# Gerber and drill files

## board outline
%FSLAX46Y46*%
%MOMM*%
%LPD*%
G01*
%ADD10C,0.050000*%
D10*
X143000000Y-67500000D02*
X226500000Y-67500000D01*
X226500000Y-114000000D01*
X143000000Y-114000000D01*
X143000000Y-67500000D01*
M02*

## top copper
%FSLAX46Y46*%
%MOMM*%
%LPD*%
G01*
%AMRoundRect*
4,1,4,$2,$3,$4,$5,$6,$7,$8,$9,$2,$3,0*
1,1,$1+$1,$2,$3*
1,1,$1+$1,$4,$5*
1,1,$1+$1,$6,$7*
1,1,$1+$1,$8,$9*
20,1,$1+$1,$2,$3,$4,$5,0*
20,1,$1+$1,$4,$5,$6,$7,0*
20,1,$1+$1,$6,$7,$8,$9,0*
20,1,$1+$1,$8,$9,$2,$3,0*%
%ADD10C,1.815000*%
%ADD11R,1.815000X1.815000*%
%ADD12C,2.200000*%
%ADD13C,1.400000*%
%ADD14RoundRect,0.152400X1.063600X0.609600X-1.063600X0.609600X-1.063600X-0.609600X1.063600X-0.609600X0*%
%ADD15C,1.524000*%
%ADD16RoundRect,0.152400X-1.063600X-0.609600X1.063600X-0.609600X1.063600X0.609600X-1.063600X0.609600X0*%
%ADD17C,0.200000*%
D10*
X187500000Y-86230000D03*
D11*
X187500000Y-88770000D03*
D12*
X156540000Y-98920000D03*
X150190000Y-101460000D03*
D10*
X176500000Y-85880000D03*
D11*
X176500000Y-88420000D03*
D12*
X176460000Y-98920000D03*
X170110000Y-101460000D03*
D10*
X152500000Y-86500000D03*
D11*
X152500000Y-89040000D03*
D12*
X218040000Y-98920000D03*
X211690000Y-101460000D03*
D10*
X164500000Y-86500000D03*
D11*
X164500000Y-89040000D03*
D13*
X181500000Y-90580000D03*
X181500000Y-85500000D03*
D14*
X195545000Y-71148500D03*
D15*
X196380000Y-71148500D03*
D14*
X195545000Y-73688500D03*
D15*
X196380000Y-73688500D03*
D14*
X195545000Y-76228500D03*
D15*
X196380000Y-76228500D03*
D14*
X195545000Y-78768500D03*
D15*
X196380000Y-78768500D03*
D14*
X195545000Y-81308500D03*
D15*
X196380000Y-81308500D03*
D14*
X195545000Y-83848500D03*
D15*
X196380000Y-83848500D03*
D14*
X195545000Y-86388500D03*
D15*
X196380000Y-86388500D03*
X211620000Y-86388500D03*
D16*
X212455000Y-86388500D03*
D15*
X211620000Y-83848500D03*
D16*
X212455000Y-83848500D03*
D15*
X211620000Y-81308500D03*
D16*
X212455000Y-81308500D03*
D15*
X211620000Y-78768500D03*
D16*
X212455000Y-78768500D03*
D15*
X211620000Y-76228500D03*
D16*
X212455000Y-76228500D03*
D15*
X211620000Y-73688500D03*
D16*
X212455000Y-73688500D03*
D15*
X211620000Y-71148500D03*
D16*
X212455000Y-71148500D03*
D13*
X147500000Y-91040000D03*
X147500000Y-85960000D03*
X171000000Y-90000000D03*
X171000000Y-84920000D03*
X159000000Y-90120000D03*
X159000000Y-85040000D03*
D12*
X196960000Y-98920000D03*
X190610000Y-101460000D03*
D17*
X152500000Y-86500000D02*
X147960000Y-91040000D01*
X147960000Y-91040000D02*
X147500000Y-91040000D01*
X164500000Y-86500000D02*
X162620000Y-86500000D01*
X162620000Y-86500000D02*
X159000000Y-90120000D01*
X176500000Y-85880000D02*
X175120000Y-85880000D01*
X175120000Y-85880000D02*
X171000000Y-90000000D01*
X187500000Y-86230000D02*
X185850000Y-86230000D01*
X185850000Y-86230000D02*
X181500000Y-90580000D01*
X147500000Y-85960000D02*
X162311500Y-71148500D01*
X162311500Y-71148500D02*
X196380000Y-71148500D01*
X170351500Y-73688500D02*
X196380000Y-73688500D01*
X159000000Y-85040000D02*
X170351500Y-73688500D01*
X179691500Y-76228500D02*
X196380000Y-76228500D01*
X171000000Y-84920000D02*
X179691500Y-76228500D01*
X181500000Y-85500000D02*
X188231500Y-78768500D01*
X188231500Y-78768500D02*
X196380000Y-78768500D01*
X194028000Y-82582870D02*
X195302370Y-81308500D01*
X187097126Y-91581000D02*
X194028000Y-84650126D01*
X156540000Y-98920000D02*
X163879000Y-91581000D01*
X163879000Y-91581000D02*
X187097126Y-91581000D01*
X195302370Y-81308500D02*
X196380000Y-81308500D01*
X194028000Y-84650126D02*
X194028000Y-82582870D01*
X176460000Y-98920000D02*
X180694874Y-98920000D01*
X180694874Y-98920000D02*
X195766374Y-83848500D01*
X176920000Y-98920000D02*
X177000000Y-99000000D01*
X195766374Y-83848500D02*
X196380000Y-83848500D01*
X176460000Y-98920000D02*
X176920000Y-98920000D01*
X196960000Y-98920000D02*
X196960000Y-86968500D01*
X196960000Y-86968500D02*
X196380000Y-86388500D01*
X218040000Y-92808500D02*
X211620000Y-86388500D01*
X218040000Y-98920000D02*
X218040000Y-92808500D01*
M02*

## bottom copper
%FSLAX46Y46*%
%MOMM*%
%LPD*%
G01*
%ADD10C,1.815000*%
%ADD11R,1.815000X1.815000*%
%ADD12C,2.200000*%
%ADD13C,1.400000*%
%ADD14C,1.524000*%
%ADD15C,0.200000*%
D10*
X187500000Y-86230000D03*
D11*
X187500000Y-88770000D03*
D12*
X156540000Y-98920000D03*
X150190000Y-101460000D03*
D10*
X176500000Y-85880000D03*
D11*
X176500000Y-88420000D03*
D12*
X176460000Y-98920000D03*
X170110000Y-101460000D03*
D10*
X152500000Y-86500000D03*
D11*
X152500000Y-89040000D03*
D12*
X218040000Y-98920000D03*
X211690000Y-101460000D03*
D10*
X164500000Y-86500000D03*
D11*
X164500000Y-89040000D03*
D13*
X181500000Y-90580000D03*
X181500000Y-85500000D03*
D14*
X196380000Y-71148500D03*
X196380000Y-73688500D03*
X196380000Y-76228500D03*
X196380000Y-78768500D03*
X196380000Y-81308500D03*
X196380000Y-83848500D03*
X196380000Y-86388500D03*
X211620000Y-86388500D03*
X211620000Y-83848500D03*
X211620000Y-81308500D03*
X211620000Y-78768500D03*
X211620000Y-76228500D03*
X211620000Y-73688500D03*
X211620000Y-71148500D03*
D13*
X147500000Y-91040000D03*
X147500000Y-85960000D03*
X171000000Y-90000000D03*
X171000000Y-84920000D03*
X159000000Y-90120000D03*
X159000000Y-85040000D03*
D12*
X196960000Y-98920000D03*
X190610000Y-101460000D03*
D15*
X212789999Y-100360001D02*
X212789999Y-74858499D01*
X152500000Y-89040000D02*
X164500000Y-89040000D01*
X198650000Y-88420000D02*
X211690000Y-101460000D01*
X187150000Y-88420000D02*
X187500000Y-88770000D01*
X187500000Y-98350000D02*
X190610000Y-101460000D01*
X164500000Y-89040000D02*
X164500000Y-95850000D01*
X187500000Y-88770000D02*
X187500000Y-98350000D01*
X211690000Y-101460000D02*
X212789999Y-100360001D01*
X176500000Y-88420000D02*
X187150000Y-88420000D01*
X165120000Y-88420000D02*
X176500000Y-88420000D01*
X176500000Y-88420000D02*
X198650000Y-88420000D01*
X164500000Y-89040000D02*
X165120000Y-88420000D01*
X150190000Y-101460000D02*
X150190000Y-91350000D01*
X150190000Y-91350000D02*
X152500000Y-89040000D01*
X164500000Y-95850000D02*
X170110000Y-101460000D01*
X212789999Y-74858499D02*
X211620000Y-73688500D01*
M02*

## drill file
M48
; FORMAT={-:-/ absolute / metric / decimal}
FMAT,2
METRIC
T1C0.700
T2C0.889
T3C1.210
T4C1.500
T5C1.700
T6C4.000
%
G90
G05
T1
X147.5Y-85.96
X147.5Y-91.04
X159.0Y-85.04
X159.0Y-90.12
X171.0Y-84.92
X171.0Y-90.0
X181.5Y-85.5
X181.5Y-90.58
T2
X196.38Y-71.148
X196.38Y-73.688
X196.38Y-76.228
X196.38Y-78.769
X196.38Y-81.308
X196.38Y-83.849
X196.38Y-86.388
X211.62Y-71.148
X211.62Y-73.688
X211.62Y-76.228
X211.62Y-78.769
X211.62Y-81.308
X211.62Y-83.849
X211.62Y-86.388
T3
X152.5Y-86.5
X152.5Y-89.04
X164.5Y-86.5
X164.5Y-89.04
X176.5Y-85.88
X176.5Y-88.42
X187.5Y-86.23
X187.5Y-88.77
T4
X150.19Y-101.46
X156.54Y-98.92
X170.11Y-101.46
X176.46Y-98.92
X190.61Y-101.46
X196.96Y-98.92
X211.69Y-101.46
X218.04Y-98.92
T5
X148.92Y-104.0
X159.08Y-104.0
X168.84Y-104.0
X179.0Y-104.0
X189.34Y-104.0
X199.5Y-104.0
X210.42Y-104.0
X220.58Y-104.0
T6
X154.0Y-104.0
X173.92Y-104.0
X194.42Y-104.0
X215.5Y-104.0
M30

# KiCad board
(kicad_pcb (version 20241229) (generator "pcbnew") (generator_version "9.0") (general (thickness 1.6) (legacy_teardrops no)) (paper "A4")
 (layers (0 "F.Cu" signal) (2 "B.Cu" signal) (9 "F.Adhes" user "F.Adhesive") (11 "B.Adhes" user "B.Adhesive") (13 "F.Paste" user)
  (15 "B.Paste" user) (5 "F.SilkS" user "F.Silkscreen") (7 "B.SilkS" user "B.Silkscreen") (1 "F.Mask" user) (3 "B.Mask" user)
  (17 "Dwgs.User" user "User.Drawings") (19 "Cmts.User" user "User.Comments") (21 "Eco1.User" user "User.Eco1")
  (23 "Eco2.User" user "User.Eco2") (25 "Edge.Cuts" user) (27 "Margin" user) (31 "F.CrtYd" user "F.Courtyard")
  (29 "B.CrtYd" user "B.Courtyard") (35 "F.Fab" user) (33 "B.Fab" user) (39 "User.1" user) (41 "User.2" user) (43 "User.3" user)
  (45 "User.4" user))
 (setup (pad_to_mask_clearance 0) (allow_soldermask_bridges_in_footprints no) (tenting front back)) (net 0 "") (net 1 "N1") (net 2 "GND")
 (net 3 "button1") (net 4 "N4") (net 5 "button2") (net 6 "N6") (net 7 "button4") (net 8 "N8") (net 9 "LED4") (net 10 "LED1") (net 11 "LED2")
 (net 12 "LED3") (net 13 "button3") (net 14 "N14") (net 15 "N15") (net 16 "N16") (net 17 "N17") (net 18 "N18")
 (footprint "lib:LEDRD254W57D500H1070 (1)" (layer "F.Cu") (at 187.5 87.5 90)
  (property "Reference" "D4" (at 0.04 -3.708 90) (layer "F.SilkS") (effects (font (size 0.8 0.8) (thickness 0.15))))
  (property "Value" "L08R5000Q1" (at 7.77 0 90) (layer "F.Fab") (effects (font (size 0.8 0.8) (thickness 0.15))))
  (pad "A" thru_hole circle (at 1.27 0 90) (size 1.815 1.815) (drill 1.21) (layers "*.Cu" "*.Mask") (remove_unused_layers no) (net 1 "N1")
   (solder_mask_margin 0.102))
  (pad "C" thru_hole rect (at -1.27 0 90) (size 1.815 1.815) (drill 1.21) (layers "*.Cu" "*.Mask") (remove_unused_layers no) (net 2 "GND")
   (solder_mask_margin 0.102)))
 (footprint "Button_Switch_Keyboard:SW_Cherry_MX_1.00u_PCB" (layer "F.Cu") (at 156.54 98.92)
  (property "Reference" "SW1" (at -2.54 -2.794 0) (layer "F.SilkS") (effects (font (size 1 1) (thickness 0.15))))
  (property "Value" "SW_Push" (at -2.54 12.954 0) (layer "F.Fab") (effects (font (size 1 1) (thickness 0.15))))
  (pad "" np_thru_hole circle (at -7.62 5.08) (size 1.7 1.7) (drill 1.7) (layers "*.Cu" "*.Mask"))
  (pad "" np_thru_hole circle (at -2.54 5.08) (size 4 4) (drill 4) (layers "*.Cu" "*.Mask"))
  (pad "" np_thru_hole circle (at 2.54 5.08) (size 1.7 1.7) (drill 1.7) (layers "*.Cu" "*.Mask"))
  (pad "1" thru_hole circle (at 0 0) (size 2.2 2.2) (drill 1.5) (layers "*.Cu" "*.Mask") (remove_unused_layers no) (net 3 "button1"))
  (pad "2" thru_hole circle (at -6.35 2.54) (size 2.2 2.2) (drill 1.5) (layers "*.Cu" "*.Mask") (remove_unused_layers no) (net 2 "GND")))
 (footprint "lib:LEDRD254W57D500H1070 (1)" (layer "F.Cu") (at 176.5 87.15 90)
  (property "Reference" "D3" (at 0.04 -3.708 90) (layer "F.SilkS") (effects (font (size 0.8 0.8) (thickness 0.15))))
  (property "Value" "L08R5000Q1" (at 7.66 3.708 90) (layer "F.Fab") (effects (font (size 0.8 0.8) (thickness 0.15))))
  (pad "A" thru_hole circle (at 1.27 0 90) (size 1.815 1.815) (drill 1.21) (layers "*.Cu" "*.Mask") (remove_unused_layers no) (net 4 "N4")
   (solder_mask_margin 0.102))
  (pad "C" thru_hole rect (at -1.27 0 90) (size 1.815 1.815) (drill 1.21) (layers "*.Cu" "*.Mask") (remove_unused_layers no) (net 2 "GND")
   (solder_mask_margin 0.102)))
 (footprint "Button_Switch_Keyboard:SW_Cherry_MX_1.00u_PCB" (layer "F.Cu") (at 176.46 98.92)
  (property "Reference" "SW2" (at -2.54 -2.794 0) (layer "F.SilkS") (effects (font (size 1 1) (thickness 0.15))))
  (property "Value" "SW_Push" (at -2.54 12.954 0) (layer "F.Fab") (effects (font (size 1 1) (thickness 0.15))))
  (pad "" np_thru_hole circle (at -7.62 5.08) (size 1.7 1.7) (drill 1.7) (layers "*.Cu" "*.Mask"))
  (pad "" np_thru_hole circle (at -2.54 5.08) (size 4 4) (drill 4) (layers "*.Cu" "*.Mask"))
  (pad "" np_thru_hole circle (at 2.54 5.08) (size 1.7 1.7) (drill 1.7) (layers "*.Cu" "*.Mask"))
  (pad "1" thru_hole circle (at 0 0) (size 2.2 2.2) (drill 1.5) (layers "*.Cu" "*.Mask") (remove_unused_layers no) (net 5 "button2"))
  (pad "2" thru_hole circle (at -6.35 2.54) (size 2.2 2.2) (drill 1.5) (layers "*.Cu" "*.Mask") (remove_unused_layers no) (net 2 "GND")))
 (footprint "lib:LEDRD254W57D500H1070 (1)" (layer "F.Cu") (at 152.5 87.77 90)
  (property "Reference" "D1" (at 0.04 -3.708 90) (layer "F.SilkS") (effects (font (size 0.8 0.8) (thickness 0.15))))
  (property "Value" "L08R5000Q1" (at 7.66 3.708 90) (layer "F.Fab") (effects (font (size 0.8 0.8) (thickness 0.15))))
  (pad "A" thru_hole circle (at 1.27 0 90) (size 1.815 1.815) (drill 1.21) (layers "*.Cu" "*.Mask") (remove_unused_layers no) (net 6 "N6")
   (solder_mask_margin 0.102))
  (pad "C" thru_hole rect (at -1.27 0 90) (size 1.815 1.815) (drill 1.21) (layers "*.Cu" "*.Mask") (remove_unused_layers no) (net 2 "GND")
   (solder_mask_margin 0.102)))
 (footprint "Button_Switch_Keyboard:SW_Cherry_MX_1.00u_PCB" (layer "F.Cu") (at 218.04 98.92)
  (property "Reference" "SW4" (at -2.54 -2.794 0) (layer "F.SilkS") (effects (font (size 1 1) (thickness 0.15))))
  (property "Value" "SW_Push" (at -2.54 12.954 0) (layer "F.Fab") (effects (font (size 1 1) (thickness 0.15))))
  (pad "" np_thru_hole circle (at -7.62 5.08) (size 1.7 1.7) (drill 1.7) (layers "*.Cu" "*.Mask"))
  (pad "" np_thru_hole circle (at -2.54 5.08) (size 4 4) (drill 4) (layers "*.Cu" "*.Mask"))
  (pad "" np_thru_hole circle (at 2.54 5.08) (size 1.7 1.7) (drill 1.7) (layers "*.Cu" "*.Mask"))
  (pad "1" thru_hole circle (at 0 0) (size 2.2 2.2) (drill 1.5) (layers "*.Cu" "*.Mask") (remove_unused_layers no) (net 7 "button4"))
  (pad "2" thru_hole circle (at -6.35 2.54) (size 2.2 2.2) (drill 1.5) (layers "*.Cu" "*.Mask") (remove_unused_layers no) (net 2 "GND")))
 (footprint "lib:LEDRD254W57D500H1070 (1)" (layer "F.Cu") (at 164.5 87.77 90)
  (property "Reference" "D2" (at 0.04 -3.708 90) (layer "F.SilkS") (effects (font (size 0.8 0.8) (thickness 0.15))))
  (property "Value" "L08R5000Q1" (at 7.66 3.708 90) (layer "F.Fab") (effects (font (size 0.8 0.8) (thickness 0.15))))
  (pad "A" thru_hole circle (at 1.27 0 90) (size 1.815 1.815) (drill 1.21) (layers "*.Cu" "*.Mask") (remove_unused_layers no) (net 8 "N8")
   (solder_mask_margin 0.102))
  (pad "C" thru_hole rect (at -1.27 0 90) (size 1.815 1.815) (drill 1.21) (layers "*.Cu" "*.Mask") (remove_unused_layers no) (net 2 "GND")
   (solder_mask_margin 0.102)))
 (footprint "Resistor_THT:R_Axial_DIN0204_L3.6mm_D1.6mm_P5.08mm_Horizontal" (layer "F.Cu") (at 181.5 90.58 90)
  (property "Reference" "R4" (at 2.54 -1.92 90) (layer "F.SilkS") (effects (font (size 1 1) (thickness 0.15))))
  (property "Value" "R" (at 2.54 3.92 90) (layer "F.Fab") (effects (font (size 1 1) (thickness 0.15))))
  (pad "1" thru_hole circle (at 0 0 90) (size 1.4 1.4) (drill 0.7) (layers "*.Cu" "*.Mask") (remove_unused_layers no) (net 1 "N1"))
  (pad "2" thru_hole circle (at 5.08 0 90) (size 1.4 1.4) (drill 0.7) (layers "*.Cu" "*.Mask") (remove_unused_layers no) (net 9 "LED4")))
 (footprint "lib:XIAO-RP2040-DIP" (layer "F.Cu") (at 204 78.7685)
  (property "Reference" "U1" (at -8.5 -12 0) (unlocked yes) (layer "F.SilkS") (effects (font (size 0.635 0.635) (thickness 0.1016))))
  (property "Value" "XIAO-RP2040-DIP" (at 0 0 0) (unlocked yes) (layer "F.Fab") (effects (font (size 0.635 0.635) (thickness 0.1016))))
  (pad "1" smd roundrect (at -8.455 -7.62 180) (size 2.432 1.524) (layers "F.Cu" "F.Mask") (roundrect_rratio 0.1) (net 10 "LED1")
   (thermal_bridge_angle 45))
  (pad "1" thru_hole circle (at -7.62 -7.62 180) (size 1.524 1.524) (drill 0.889) (layers "*.Cu" "*.Mask") (remove_unused_layers no)
   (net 10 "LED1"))
  (pad "2" smd roundrect (at -8.455 -5.08 180) (size 2.432 1.524) (layers "F.Cu" "F.Mask") (roundrect_rratio 0.1) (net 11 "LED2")
   (thermal_bridge_angle 45))
  (pad "2" thru_hole circle (at -7.62 -5.08 180) (size 1.524 1.524) (drill 0.889) (layers "*.Cu" "*.Mask") (remove_unused_layers no)
   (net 11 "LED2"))
  (pad "3" smd roundrect (at -8.455 -2.54 180) (size 2.432 1.524) (layers "F.Cu" "F.Mask") (roundrect_rratio 0.1) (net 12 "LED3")
   (thermal_bridge_angle 45))
  (pad "3" thru_hole circle (at -7.62 -2.54 180) (size 1.524 1.524) (drill 0.889) (layers "*.Cu" "*.Mask") (remove_unused_layers no)
   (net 12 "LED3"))
  (pad "4" smd roundrect (at -8.455 0 180) (size 2.432 1.524) (layers "F.Cu" "F.Mask") (roundrect_rratio 0.1) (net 9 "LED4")
   (thermal_bridge_angle 45))
  (pad "4" thru_hole circle (at -7.62 0 180) (size 1.524 1.524) (drill 0.889) (layers "*.Cu" "*.Mask") (remove_unused_layers no)
   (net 9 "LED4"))
  (pad "5" smd roundrect (at -8.455 2.54 180) (size 2.432 1.524) (layers "F.Cu" "F.Mask") (roundrect_rratio 0.1) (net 3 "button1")
   (thermal_bridge_angle 45))
  (pad "5" thru_hole circle (at -7.62 2.54 180) (size 1.524 1.524) (drill 0.889) (layers "*.Cu" "*.Mask") (remove_unused_layers no)
   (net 3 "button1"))
  (pad "6" smd roundrect (at -8.455 5.08 180) (size 2.432 1.524) (layers "F.Cu" "F.Mask") (roundrect_rratio 0.1) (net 5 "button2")
   (thermal_bridge_angle 45))
  (pad "6" thru_hole circle (at -7.62 5.08 180) (size 1.524 1.524) (drill 0.889) (layers "*.Cu" "*.Mask") (remove_unused_layers no)
   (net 5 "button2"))
  (pad "7" smd roundrect (at -8.455 7.62 180) (size 2.432 1.524) (layers "F.Cu" "F.Mask") (roundrect_rratio 0.1) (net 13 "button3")
   (thermal_bridge_angle 45))
  (pad "7" thru_hole circle (at -7.62 7.62 180) (size 1.524 1.524) (drill 0.889) (layers "*.Cu" "*.Mask") (remove_unused_layers no)
   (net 13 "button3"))
  (pad "8" thru_hole circle (at 7.62 7.62) (size 1.524 1.524) (drill 0.889) (layers "*.Cu" "*.Mask") (remove_unused_layers no)
   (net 7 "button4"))
  (pad "8" smd roundrect (at 8.455 7.62) (size 2.432 1.524) (layers "F.Cu" "F.Mask") (roundrect_rratio 0.1) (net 7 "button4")
   (thermal_bridge_angle 45))
  (pad "9" thru_hole circle (at 7.62 5.08) (size 1.524 1.524) (drill 0.889) (layers "*.Cu" "*.Mask") (remove_unused_layers no)
   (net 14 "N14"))
  (pad "9" smd roundrect (at 8.455 5.08) (size 2.432 1.524) (layers "F.Cu" "F.Mask") (roundrect_rratio 0.1) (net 14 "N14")
   (thermal_bridge_angle 45))
  (pad "10" thru_hole circle (at 7.62 2.54) (size 1.524 1.524) (drill 0.889) (layers "*.Cu" "*.Mask") (remove_unused_layers no)
   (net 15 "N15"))
  (pad "10" smd roundrect (at 8.455 2.54) (size 2.432 1.524) (layers "F.Cu" "F.Mask") (roundrect_rratio 0.1) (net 15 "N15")
   (thermal_bridge_angle 45))
  (pad "11" thru_hole circle (at 7.62 0) (size 1.524 1.524) (drill 0.889) (layers "*.Cu" "*.Mask") (remove_unused_layers no) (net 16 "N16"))
  (pad "11" smd roundrect (at 8.455 0) (size 2.432 1.524) (layers "F.Cu" "F.Mask") (roundrect_rratio 0.1) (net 16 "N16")
   (thermal_bridge_angle 45))
  (pad "12" thru_hole circle (at 7.62 -2.54) (size 1.524 1.524) (drill 0.889) (layers "*.Cu" "*.Mask") (remove_unused_layers no)
   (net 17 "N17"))
  (pad "12" smd roundrect (at 8.455 -2.54) (size 2.432 1.524) (layers "F.Cu" "F.Mask") (roundrect_rratio 0.1) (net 17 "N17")
   (thermal_bridge_angle 45))
  (pad "13" thru_hole circle (at 7.62 -5.08) (size 1.524 1.524) (drill 0.889) (layers "*.Cu" "*.Mask") (remove_unused_layers no)
   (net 2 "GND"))
  (pad "13" smd roundrect (at 8.455 -5.08) (size 2.432 1.524) (layers "F.Cu" "F.Mask") (roundrect_rratio 0.1) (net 2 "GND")
   (thermal_bridge_angle 45))
  (pad "14" thru_hole circle (at 7.62 -7.62) (size 1.524 1.524) (drill 0.889) (layers "*.Cu" "*.Mask") (remove_unused_layers no)
   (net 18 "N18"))
  (pad "14" smd roundrect (at 8.455 -7.62) (size 2.432 1.524) (layers "F.Cu" "F.Mask") (roundrect_rratio 0.1) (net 18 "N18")
   (thermal_bridge_angle 45)))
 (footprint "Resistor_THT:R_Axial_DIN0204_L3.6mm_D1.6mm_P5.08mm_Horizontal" (layer "F.Cu") (at 147.5 91.04 90)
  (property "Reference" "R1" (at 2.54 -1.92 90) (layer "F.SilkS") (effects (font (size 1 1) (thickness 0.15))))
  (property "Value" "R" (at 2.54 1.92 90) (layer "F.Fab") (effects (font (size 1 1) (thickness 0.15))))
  (pad "1" thru_hole circle (at 0 0 90) (size 1.4 1.4) (drill 0.7) (layers "*.Cu" "*.Mask") (remove_unused_layers no) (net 6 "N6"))
  (pad "2" thru_hole circle (at 5.08 0 90) (size 1.4 1.4) (drill 0.7) (layers "*.Cu" "*.Mask") (remove_unused_layers no) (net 10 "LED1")))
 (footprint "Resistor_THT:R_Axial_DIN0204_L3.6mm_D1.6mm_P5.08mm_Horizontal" (layer "F.Cu") (at 171 90 90)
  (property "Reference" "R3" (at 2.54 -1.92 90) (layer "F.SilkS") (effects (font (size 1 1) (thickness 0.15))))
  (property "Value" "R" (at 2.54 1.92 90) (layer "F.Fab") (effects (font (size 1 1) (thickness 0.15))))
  (pad "1" thru_hole circle (at 0 0 90) (size 1.4 1.4) (drill 0.7) (layers "*.Cu" "*.Mask") (remove_unused_layers no) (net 4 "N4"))
  (pad "2" thru_hole circle (at 5.08 0 90) (size 1.4 1.4) (drill 0.7) (layers "*.Cu" "*.Mask") (remove_unused_layers no) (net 12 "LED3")))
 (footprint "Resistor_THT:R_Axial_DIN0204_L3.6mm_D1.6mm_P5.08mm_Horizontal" (layer "F.Cu") (at 159 90.12 90)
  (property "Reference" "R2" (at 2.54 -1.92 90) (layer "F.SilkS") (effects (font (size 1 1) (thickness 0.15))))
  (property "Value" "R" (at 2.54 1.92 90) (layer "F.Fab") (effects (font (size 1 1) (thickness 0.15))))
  (pad "1" thru_hole circle (at 0 0 90) (size 1.4 1.4) (drill 0.7) (layers "*.Cu" "*.Mask") (remove_unused_layers no) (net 8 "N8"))
  (pad "2" thru_hole circle (at 5.08 0 90) (size 1.4 1.4) (drill 0.7) (layers "*.Cu" "*.Mask") (remove_unused_layers no) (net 11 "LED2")))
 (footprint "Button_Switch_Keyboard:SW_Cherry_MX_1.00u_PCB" (layer "F.Cu") (at 196.96 98.92)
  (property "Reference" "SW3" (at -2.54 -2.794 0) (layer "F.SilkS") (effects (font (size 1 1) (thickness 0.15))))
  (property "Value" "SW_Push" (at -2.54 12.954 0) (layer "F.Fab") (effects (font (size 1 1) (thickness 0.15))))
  (pad "" np_thru_hole circle (at -7.62 5.08) (size 1.7 1.7) (drill 1.7) (layers "*.Cu" "*.Mask"))
  (pad "" np_thru_hole circle (at -2.54 5.08) (size 4 4) (drill 4) (layers "*.Cu" "*.Mask"))
  (pad "" np_thru_hole circle (at 2.54 5.08) (size 1.7 1.7) (drill 1.7) (layers "*.Cu" "*.Mask"))
  (pad "1" thru_hole circle (at 0 0) (size 2.2 2.2) (drill 1.5) (layers "*.Cu" "*.Mask") (remove_unused_layers no) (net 13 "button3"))
  (pad "2" thru_hole circle (at -6.35 2.54) (size 2.2 2.2) (drill 1.5) (layers "*.Cu" "*.Mask") (remove_unused_layers no) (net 2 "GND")))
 (gr_rect (start 143 67.5) (end 226.5 114) (stroke (width 0.05) (type default)) (fill no) (layer "Edge.Cuts"))
 (segment (start 152.5 86.5) (end 147.96 91.04) (width 0.2) (layer "F.Cu") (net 6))
 (segment (start 147.96 91.04) (end 147.5 91.04) (width 0.2) (layer "F.Cu") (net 6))
 (segment (start 212.789999 100.360001) (end 212.789999 74.858499) (width 0.2) (layer "B.Cu") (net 2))
 (segment (start 152.5 89.04) (end 164.5 89.04) (width 0.2) (layer "B.Cu") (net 2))
 (segment (start 198.65 88.42) (end 211.69 101.46) (width 0.2) (layer "B.Cu") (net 2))
 (segment (start 187.15 88.42) (end 187.5 88.77) (width 0.2) (layer "B.Cu") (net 2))
 (segment (start 187.5 98.35) (end 190.61 101.46) (width 0.2) (layer "B.Cu") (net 2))
 (segment (start 164.5 89.04) (end 164.5 95.85) (width 0.2) (layer "B.Cu") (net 2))
 (segment (start 187.5 88.77) (end 187.5 98.35) (width 0.2) (layer "B.Cu") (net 2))
 (segment (start 211.69 101.46) (end 212.789999 100.360001) (width 0.2) (layer "B.Cu") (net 2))
 (segment (start 176.5 88.42) (end 187.15 88.42) (width 0.2) (layer "B.Cu") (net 2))
 (segment (start 165.12 88.42) (end 176.5 88.42) (width 0.2) (layer "B.Cu") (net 2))
 (segment (start 176.5 88.42) (end 198.65 88.42) (width 0.2) (layer "B.Cu") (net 2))
 (segment (start 164.5 89.04) (end 165.12 88.42) (width 0.2) (layer "B.Cu") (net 2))
 (segment (start 150.19 101.46) (end 150.19 91.35) (width 0.2) (layer "B.Cu") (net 2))
 (segment (start 150.19 91.35) (end 152.5 89.04) (width 0.2) (layer "B.Cu") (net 2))
 (segment (start 164.5 95.85) (end 170.11 101.46) (width 0.2) (layer "B.Cu") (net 2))
 (segment (start 212.789999 74.858499) (end 211.62 73.6885) (width 0.2) (layer "B.Cu") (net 2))
 (segment (start 164.5 86.5) (end 162.62 86.5) (width 0.2) (layer "F.Cu") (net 8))
 (segment (start 162.62 86.5) (end 159 90.12) (width 0.2) (layer "F.Cu") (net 8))
 (segment (start 176.5 85.88) (end 175.12 85.88) (width 0.2) (layer "F.Cu") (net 4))
 (segment (start 175.12 85.88) (end 171 90) (width 0.2) (layer "F.Cu") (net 4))
 (segment (start 187.5 86.23) (end 185.85 86.23) (width 0.2) (layer "F.Cu") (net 1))
 (segment (start 185.85 86.23) (end 181.5 90.58) (width 0.2) (layer "F.Cu") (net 1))
 (segment (start 147.5 85.96) (end 162.3115 71.1485) (width 0.2) (layer "F.Cu") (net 10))
 (segment (start 162.3115 71.1485) (end 196.38 71.1485) (width 0.2) (layer "F.Cu") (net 10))
 (segment (start 170.3515 73.6885) (end 196.38 73.6885) (width 0.2) (layer "F.Cu") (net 11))
 (segment (start 159 85.04) (end 170.3515 73.6885) (width 0.2) (layer "F.Cu") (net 11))
 (segment (start 179.6915 76.2285) (end 196.38 76.2285) (width 0.2) (layer "F.Cu") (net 12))
 (segment (start 171 84.92) (end 179.6915 76.2285) (width 0.2) (layer "F.Cu") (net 12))
 (segment (start 181.5 85.5) (end 188.2315 78.7685) (width 0.2) (layer "F.Cu") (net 9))
 (segment (start 188.2315 78.7685) (end 196.38 78.7685) (width 0.2) (layer "F.Cu") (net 9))
 (segment (start 194.028 82.58287) (end 195.30237 81.3085) (width 0.2) (layer "F.Cu") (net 3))
 (segment (start 187.097126 91.581) (end 194.028 84.650126) (width 0.2) (layer "F.Cu") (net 3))
 (segment (start 156.54 98.92) (end 163.879 91.581) (width 0.2) (layer "F.Cu") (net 3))
 (segment (start 163.879 91.581) (end 187.097126 91.581) (width 0.2) (layer "F.Cu") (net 3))
 (segment (start 195.30237 81.3085) (end 196.38 81.3085) (width 0.2) (layer "F.Cu") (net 3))
 (segment (start 194.028 84.650126) (end 194.028 82.58287) (width 0.2) (layer "F.Cu") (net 3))
 (segment (start 176.46 98.92) (end 180.694874 98.92) (width 0.2) (layer "F.Cu") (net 5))
 (segment (start 180.694874 98.92) (end 195.766374 83.8485) (width 0.2) (layer "F.Cu") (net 5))
 (segment (start 176.92 98.92) (end 177 99) (width 0.2) (layer "F.Cu") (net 5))
 (segment (start 195.766374 83.8485) (end 196.38 83.8485) (width 0.2) (layer "F.Cu") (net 5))
 (segment (start 176.46 98.92) (end 176.92 98.92) (width 0.2) (layer "F.Cu") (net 5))
 (segment (start 196.96 98.92) (end 196.96 86.9685) (width 0.2) (layer "F.Cu") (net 13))
 (segment (start 196.96 86.9685) (end 196.38 86.3885) (width 0.2) (layer "F.Cu") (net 13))
 (segment (start 218.04 92.8085) (end 211.62 86.3885) (width 0.2) (layer "F.Cu") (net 7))
 (segment (start 218.04 98.92) (end 218.04 92.8085) (width 0.2) (layer "F.Cu") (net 7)))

